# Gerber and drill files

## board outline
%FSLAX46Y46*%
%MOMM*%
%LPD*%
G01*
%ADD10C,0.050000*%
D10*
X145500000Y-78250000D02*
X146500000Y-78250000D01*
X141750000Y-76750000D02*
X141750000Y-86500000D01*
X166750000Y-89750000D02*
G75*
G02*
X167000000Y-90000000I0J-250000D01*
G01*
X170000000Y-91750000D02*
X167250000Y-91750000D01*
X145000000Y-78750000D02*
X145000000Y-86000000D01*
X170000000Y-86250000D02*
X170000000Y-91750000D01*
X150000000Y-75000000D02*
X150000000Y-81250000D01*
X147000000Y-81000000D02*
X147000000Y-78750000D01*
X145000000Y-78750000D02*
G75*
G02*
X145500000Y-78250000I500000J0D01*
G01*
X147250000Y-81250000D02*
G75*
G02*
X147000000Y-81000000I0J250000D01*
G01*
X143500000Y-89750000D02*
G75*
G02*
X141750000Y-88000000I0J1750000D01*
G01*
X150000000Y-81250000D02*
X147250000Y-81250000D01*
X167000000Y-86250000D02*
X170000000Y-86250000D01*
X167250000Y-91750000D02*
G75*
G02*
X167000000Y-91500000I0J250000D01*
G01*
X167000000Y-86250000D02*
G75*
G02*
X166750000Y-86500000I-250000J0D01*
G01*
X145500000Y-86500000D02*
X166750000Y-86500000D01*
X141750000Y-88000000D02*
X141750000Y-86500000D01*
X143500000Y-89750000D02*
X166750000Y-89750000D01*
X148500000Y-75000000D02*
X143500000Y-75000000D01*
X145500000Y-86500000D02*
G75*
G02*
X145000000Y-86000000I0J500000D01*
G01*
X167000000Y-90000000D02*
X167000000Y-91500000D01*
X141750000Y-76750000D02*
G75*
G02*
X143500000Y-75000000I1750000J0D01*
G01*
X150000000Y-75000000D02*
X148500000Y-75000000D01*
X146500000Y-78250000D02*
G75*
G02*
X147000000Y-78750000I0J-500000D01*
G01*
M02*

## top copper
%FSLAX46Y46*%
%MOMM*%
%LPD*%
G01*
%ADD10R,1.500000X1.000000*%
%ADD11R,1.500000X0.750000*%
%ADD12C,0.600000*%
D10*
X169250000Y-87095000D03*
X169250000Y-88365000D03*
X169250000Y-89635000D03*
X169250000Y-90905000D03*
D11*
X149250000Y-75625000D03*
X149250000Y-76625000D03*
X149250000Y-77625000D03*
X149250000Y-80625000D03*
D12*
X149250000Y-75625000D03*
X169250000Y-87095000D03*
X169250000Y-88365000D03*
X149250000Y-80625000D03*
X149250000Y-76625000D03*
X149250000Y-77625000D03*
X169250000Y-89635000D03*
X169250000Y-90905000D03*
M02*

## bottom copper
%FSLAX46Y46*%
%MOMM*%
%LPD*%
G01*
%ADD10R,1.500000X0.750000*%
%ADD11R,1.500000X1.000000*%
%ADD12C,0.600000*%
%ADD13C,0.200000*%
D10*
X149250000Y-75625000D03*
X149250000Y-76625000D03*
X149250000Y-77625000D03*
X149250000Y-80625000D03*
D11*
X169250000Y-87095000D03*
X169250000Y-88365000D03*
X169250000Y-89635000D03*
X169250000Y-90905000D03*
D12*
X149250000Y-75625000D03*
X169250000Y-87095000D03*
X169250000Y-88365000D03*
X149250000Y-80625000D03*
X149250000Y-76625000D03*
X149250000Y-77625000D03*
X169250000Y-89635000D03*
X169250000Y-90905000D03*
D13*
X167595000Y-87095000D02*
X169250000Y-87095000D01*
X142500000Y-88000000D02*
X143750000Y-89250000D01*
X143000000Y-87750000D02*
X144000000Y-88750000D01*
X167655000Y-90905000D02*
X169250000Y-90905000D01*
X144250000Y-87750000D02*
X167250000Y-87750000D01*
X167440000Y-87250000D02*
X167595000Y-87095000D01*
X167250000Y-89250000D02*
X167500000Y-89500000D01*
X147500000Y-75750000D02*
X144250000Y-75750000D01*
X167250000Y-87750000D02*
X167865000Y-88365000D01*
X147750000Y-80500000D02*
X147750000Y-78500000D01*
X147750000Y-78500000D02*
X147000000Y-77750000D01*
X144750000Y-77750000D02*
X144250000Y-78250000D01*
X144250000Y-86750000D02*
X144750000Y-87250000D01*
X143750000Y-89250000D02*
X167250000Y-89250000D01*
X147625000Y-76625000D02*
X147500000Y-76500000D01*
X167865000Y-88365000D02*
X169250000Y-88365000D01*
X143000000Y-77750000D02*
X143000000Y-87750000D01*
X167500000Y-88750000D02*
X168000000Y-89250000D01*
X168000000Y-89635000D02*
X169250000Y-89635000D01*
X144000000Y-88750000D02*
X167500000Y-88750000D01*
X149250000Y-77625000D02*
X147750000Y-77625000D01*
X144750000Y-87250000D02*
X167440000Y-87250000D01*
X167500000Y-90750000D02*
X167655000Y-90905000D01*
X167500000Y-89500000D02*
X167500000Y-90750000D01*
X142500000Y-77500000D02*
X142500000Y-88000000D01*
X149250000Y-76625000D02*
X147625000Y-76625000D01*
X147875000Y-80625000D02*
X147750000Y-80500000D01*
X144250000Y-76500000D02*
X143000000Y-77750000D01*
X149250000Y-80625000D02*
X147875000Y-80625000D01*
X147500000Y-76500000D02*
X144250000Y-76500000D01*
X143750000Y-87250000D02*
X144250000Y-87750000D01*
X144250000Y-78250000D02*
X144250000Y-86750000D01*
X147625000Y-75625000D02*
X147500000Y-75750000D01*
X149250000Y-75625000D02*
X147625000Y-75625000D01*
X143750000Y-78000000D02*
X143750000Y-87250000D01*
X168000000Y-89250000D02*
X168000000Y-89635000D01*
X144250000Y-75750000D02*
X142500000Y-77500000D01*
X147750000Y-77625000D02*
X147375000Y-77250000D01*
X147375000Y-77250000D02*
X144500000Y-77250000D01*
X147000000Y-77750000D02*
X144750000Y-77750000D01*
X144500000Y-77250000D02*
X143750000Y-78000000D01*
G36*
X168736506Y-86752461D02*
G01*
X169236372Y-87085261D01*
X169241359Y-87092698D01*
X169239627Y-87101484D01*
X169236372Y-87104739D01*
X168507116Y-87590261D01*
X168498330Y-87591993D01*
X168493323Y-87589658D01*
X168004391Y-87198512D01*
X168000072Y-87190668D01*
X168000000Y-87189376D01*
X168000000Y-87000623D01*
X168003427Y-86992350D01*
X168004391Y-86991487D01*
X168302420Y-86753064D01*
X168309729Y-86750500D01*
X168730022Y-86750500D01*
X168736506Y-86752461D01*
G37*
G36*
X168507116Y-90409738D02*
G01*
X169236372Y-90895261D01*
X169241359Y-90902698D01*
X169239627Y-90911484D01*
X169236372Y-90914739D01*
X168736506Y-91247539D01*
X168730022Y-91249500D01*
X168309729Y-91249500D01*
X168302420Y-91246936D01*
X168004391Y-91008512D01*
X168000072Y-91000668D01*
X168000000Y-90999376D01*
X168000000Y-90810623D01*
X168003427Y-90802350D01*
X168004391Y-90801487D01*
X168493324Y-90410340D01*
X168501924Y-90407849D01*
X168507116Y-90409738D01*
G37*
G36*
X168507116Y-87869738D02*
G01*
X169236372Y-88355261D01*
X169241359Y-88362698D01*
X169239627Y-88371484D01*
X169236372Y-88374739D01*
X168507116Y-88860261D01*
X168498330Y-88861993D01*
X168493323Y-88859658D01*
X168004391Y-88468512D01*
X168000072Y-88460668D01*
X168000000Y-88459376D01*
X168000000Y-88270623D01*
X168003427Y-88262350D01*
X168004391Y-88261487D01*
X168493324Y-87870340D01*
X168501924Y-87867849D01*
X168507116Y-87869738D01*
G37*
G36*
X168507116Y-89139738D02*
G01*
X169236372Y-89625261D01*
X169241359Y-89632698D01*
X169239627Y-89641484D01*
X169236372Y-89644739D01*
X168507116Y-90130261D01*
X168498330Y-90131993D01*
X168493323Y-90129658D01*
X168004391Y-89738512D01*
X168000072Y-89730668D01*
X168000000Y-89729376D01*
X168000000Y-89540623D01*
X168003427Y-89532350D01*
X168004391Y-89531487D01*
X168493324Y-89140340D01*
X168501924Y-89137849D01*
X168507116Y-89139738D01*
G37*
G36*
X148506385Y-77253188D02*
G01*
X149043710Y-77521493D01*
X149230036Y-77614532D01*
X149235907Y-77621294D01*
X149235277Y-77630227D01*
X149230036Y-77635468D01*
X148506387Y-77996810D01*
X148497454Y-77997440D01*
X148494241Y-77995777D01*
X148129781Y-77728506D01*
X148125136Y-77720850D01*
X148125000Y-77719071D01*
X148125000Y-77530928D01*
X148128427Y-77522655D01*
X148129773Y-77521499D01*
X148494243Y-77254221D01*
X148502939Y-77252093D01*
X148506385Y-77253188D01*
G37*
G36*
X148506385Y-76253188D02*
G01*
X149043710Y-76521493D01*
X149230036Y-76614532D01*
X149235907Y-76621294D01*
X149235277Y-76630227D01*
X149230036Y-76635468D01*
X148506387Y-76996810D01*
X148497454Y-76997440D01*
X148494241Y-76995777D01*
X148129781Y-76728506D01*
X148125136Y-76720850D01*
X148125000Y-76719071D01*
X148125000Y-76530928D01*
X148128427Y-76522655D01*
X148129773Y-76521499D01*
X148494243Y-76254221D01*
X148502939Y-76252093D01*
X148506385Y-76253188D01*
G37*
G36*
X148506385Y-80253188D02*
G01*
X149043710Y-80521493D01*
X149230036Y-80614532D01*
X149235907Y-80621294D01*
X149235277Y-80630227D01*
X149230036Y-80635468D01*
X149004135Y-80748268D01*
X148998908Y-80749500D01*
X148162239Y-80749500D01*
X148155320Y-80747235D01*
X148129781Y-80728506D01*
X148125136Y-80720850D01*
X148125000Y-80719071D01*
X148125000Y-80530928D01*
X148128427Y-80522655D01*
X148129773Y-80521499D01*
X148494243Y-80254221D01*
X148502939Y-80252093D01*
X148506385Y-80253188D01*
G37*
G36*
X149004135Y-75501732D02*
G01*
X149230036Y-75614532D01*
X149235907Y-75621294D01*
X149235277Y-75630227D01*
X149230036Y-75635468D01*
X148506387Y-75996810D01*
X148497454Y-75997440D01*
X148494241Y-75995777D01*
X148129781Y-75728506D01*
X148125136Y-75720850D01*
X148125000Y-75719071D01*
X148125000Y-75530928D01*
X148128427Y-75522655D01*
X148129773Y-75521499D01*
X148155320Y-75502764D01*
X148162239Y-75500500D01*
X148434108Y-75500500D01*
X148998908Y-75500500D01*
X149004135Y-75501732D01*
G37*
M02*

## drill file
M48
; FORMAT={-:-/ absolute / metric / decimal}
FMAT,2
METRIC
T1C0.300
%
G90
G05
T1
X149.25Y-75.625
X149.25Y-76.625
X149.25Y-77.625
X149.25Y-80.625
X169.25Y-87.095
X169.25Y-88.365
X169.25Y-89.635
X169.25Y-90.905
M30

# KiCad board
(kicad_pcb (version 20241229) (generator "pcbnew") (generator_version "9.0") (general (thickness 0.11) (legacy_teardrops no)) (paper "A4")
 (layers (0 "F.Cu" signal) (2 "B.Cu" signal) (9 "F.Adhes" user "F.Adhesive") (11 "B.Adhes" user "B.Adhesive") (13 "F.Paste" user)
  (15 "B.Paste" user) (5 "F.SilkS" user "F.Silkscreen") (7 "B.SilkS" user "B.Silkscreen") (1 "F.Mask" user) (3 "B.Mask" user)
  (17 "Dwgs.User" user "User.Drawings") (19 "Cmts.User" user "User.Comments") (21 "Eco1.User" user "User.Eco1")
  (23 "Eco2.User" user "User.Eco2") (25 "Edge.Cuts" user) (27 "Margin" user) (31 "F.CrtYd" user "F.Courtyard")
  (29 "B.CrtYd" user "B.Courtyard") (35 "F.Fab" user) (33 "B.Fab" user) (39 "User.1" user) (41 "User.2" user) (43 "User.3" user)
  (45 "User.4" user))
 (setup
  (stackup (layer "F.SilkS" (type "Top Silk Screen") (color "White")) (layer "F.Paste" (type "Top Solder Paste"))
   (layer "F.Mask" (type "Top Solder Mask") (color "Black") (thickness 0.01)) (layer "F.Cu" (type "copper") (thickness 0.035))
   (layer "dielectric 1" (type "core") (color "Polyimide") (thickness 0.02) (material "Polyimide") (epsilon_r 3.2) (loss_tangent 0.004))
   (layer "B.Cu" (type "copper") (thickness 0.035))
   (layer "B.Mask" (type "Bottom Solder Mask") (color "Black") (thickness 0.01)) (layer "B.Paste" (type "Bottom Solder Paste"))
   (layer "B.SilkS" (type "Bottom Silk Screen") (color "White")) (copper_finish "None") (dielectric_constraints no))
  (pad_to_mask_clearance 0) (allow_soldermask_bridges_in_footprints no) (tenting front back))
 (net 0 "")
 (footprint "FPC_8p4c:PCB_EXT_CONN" (layer "F.Cu") (at 169.25 89)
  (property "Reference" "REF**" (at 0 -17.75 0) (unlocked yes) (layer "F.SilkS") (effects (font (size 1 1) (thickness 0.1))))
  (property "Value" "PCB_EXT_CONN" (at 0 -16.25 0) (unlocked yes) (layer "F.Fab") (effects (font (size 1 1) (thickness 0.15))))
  (pad "1" smd rect (at 0 -1.905) (size 1.5 1) (layers "F.Cu" "F.Mask" "F.Paste")
   (teardrops (best_length_ratio 0.5) (max_length 1) (best_width_ratio 1) (max_width 2) (curved_edges no) (filter_ratio 0.9) (enabled yes)
    (allow_two_segments yes) (prefer_zone_connections yes)))
  (pad "2" smd rect (at 0 -0.635) (size 1.5 1) (layers "F.Cu" "F.Mask" "F.Paste")
   (teardrops (best_length_ratio 0.5) (max_length 1) (best_width_ratio 1) (max_width 2) (curved_edges no) (filter_ratio 0.9) (enabled yes)
    (allow_two_segments yes) (prefer_zone_connections yes)))
  (pad "3" smd rect (at 0 0.635) (size 1.5 1) (layers "F.Cu" "F.Mask" "F.Paste")
   (teardrops (best_length_ratio 0.5) (max_length 1) (best_width_ratio 1) (max_width 2) (curved_edges no) (filter_ratio 0.9) (enabled yes)
    (allow_two_segments yes) (prefer_zone_connections yes)))
  (pad "4" smd rect (at 0 1.905) (size 1.5 1) (layers "F.Cu" "F.Mask" "F.Paste")
   (teardrops (best_length_ratio 0.5) (max_length 1) (best_width_ratio 1) (max_width 2) (curved_edges no) (filter_ratio 0.9) (enabled yes)
    (allow_two_segments yes) (prefer_zone_connections yes))))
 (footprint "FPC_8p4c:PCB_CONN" (layer "F.Cu") (at 149.25 78.125)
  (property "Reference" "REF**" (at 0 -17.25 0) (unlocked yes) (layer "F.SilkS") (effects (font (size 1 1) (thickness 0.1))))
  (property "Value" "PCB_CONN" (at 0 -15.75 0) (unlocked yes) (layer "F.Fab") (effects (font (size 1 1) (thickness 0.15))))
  (pad "1" smd rect (at 0 -2.5) (size 1.5 0.75) (layers "F.Cu" "F.Mask" "F.Paste")
   (teardrops (best_length_ratio 0.5) (max_length 1) (best_width_ratio 1) (max_width 2) (curved_edges no) (filter_ratio 0.9) (enabled yes)
    (allow_two_segments yes) (prefer_zone_connections yes)))
  (pad "2" smd rect (at 0 -1.5) (size 1.5 0.75) (layers "F.Cu" "F.Mask" "F.Paste")
   (teardrops (best_length_ratio 0.5) (max_length 1) (best_width_ratio 1) (max_width 2) (curved_edges no) (filter_ratio 0.9) (enabled yes)
    (allow_two_segments yes) (prefer_zone_connections yes)))
  (pad "3" smd rect (at 0 -0.5) (size 1.5 0.75) (layers "F.Cu" "F.Mask" "F.Paste")
   (teardrops (best_length_ratio 0.5) (max_length 1) (best_width_ratio 1) (max_width 2) (curved_edges no) (filter_ratio 0.9) (enabled yes)
    (allow_two_segments yes) (prefer_zone_connections yes)))
  (pad "4" smd rect (at 0 2.5) (size 1.5 0.75) (layers "F.Cu" "F.Mask" "F.Paste")
   (teardrops (best_length_ratio 0.5) (max_length 1) (best_width_ratio 1) (max_width 2) (curved_edges no) (filter_ratio 0.9) (enabled yes)
    (allow_two_segments yes) (prefer_zone_connections yes))))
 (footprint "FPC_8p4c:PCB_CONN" (layer "B.Cu") (at 149.25 78.125 180)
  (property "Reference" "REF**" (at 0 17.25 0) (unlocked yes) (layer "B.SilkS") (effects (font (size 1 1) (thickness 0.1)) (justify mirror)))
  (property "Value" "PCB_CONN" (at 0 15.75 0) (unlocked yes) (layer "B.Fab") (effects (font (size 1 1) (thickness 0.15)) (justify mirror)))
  (pad "1" smd rect (at 0 2.5 180) (size 1.5 0.75) (layers "B.Cu" "B.Mask" "B.Paste")
   (teardrops (best_length_ratio 0.5) (max_length 1) (best_width_ratio 1) (max_width 2) (curved_edges no) (filter_ratio 0.9) (enabled yes)
    (allow_two_segments yes) (prefer_zone_connections yes)))
  (pad "2" smd rect (at 0 1.5 180) (size 1.5 0.75) (layers "B.Cu" "B.Mask" "B.Paste")
   (teardrops (best_length_ratio 0.5) (max_length 1) (best_width_ratio 1) (max_width 2) (curved_edges no) (filter_ratio 0.9) (enabled yes)
    (allow_two_segments yes) (prefer_zone_connections yes)))
  (pad "3" smd rect (at 0 0.5 180) (size 1.5 0.75) (layers "B.Cu" "B.Mask" "B.Paste")
   (teardrops (best_length_ratio 0.5) (max_length 1) (best_width_ratio 1) (max_width 2) (curved_edges no) (filter_ratio 0.9) (enabled yes)
    (allow_two_segments yes) (prefer_zone_connections yes)))
  (pad "4" smd rect (at 0 -2.5 180) (size 1.5 0.75) (layers "B.Cu" "B.Mask" "B.Paste")
   (teardrops (best_length_ratio 0.5) (max_length 1) (best_width_ratio 1) (max_width 2) (curved_edges no) (filter_ratio 0.9) (enabled yes)
    (allow_two_segments yes) (prefer_zone_connections yes))))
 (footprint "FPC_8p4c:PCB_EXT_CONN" (layer "B.Cu") (at 169.25 89 180)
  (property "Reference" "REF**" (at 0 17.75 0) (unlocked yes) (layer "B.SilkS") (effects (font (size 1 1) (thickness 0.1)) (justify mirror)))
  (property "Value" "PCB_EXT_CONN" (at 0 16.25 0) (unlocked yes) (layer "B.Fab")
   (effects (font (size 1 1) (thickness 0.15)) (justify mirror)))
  (pad "1" smd rect (at 0 1.905 180) (size 1.5 1) (layers "B.Cu" "B.Mask" "B.Paste")
   (teardrops (best_length_ratio 0.5) (max_length 1) (best_width_ratio 1) (max_width 2) (curved_edges no) (filter_ratio 0.9) (enabled yes)
    (allow_two_segments yes) (prefer_zone_connections yes)))
  (pad "2" smd rect (at 0 0.635 180) (size 1.5 1) (layers "B.Cu" "B.Mask" "B.Paste")
   (teardrops (best_length_ratio 0.5) (max_length 1) (best_width_ratio 1) (max_width 2) (curved_edges no) (filter_ratio 0.9) (enabled yes)
    (allow_two_segments yes) (prefer_zone_connections yes)))
  (pad "3" smd rect (at 0 -0.635 180) (size 1.5 1) (layers "B.Cu" "B.Mask" "B.Paste")
   (teardrops (best_length_ratio 0.5) (max_length 1) (best_width_ratio 1) (max_width 2) (curved_edges no) (filter_ratio 0.9) (enabled yes)
    (allow_two_segments yes) (prefer_zone_connections yes)))
  (pad "4" smd rect (at 0 -1.905 180) (size 1.5 1) (layers "B.Cu" "B.Mask" "B.Paste")
   (teardrops (best_length_ratio 0.5) (max_length 1) (best_width_ratio 1) (max_width 2) (curved_edges no) (filter_ratio 0.9) (enabled yes)
    (allow_two_segments yes) (prefer_zone_connections yes))))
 (gr_line (start 145.5 78.25) (end 146.5 78.25) (stroke (width 0.05) (type default)) (layer "Edge.Cuts"))
 (gr_line (start 141.75 76.75) (end 141.75 86.5) (stroke (width 0.05) (type default)) (layer "Edge.Cuts"))
 (gr_arc (start 166.75 89.75) (mid 166.926777 89.823223) (end 167 90) (stroke (width 0.05) (type default)) (layer "Edge.Cuts"))
 (gr_line (start 170 91.75) (end 167.25 91.75) (stroke (width 0.05) (type default)) (layer "Edge.Cuts"))
 (gr_line (start 145 78.75) (end 145 86) (stroke (width 0.05) (type default)) (layer "Edge.Cuts"))
 (gr_line (start 170 86.25) (end 170 91.75) (stroke (width 0.05) (type default)) (layer "Edge.Cuts"))
 (gr_line (start 150 75) (end 150 81.25) (stroke (width 0.05) (type default)) (layer "Edge.Cuts"))
 (gr_line (start 147 81) (end 147 78.75) (stroke (width 0.05) (type default)) (layer "Edge.Cuts"))
 (gr_arc (start 145 78.75) (mid 145.146447 78.396447) (end 145.5 78.25) (stroke (width 0.05) (type default)) (layer "Edge.Cuts"))
 (gr_arc (start 147.25 81.25) (mid 147.073223 81.176777) (end 147 81) (stroke (width 0.05) (type default)) (layer "Edge.Cuts"))
 (gr_arc (start 143.5 89.75) (mid 142.262563 89.237437) (end 141.75 88) (stroke (width 0.05) (type default)) (layer "Edge.Cuts"))
 (gr_line (start 150 81.25) (end 147.25 81.25) (stroke (width 0.05) (type default)) (layer "Edge.Cuts"))
 (gr_line (start 167 86.25) (end 170 86.25) (stroke (width 0.05) (type default)) (layer "Edge.Cuts"))
 (gr_arc (start 167.25 91.75) (mid 167.073223 91.676777) (end 167 91.5) (stroke (width 0.05) (type default)) (layer "Edge.Cuts"))
 (gr_arc (start 167 86.25) (mid 166.926777 86.426777) (end 166.75 86.5) (stroke (width 0.05) (type default)) (layer "Edge.Cuts"))
 (gr_line (start 145.5 86.5) (end 166.75 86.5) (stroke (width 0.05) (type default)) (layer "Edge.Cuts"))
 (gr_line (start 141.75 88) (end 141.75 86.5) (stroke (width 0.05) (type default)) (layer "Edge.Cuts"))
 (gr_line (start 143.5 89.75) (end 166.75 89.75) (stroke (width 0.05) (type default)) (layer "Edge.Cuts"))
 (gr_line (start 148.5 75) (end 143.5 75) (stroke (width 0.05) (type default)) (layer "Edge.Cuts"))
 (gr_arc (start 145.5 86.5) (mid 145.146447 86.353553) (end 145 86) (stroke (width 0.05) (type default)) (layer "Edge.Cuts"))
 (gr_line (start 167 90) (end 167 91.5) (stroke (width 0.05) (type default)) (layer "Edge.Cuts"))
 (gr_arc (start 141.75 76.75) (mid 142.262563 75.512563) (end 143.5 75) (stroke (width 0.05) (type default)) (layer "Edge.Cuts"))
 (gr_line (start 150 75) (end 148.5 75) (stroke (width 0.05) (type default)) (layer "Edge.Cuts"))
 (gr_arc (start 146.5 78.25) (mid 146.853553 78.396447) (end 147 78.75) (stroke (width 0.05) (type default)) (layer "Edge.Cuts"))
 (via (at 149.25 75.625) (size 0.6) (drill 0.3) (layers "F.Cu" "B.Cu") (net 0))
 (via (at 169.25 87.095) (size 0.6) (drill 0.3) (layers "F.Cu" "B.Cu") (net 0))
 (via (at 169.25 88.365) (size 0.6) (drill 0.3) (layers "F.Cu" "B.Cu") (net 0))
 (via (at 149.25 80.625) (size 0.6) (drill 0.3) (layers "F.Cu" "B.Cu") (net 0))
 (via (at 149.25 76.625) (size 0.6) (drill 0.3) (layers "F.Cu" "B.Cu") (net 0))
 (via (at 149.25 77.625) (size 0.6) (drill 0.3) (layers "F.Cu" "B.Cu") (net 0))
 (via (at 169.25 89.635) (size 0.6) (drill 0.3) (layers "F.Cu" "B.Cu") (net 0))
 (via (at 169.25 90.905) (size 0.6) (drill 0.3) (layers "F.Cu" "B.Cu") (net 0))
 (segment (start 167.595 87.095) (end 169.25 87.095) (width 0.2) (layer "B.Cu") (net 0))
 (segment (start 142.5 88) (end 143.75 89.25) (width 0.2) (layer "B.Cu") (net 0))
 (segment (start 143 87.75) (end 144 88.75) (width 0.2) (layer "B.Cu") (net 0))
 (segment (start 167.655 90.905) (end 169.25 90.905) (width 0.2) (layer "B.Cu") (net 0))
 (segment (start 144.25 87.75) (end 167.25 87.75) (width 0.2) (layer "B.Cu") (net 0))
 (segment (start 167.44 87.25) (end 167.595 87.095) (width 0.2) (layer "B.Cu") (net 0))
 (segment (start 167.25 89.25) (end 167.5 89.5) (width 0.2) (layer "B.Cu") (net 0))
 (segment (start 147.5 75.75) (end 144.25 75.75) (width 0.2) (layer "B.Cu") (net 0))
 (segment (start 167.25 87.75) (end 167.865 88.365) (width 0.2) (layer "B.Cu") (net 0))
 (segment (start 147.75 80.5) (end 147.75 78.5) (width 0.2) (layer "B.Cu") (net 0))
 (segment (start 147.75 78.5) (end 147 77.75) (width 0.2) (layer "B.Cu") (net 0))
 (segment (start 144.75 77.75) (end 144.25 78.25) (width 0.2) (layer "B.Cu") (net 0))
 (segment (start 144.25 86.75) (end 144.75 87.25) (width 0.2) (layer "B.Cu") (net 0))
 (segment (start 143.75 89.25) (end 167.25 89.25) (width 0.2) (layer "B.Cu") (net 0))
 (segment (start 147.625 76.625) (end 147.5 76.5) (width 0.2) (layer "B.Cu") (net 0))
 (segment (start 167.865 88.365) (end 169.25 88.365) (width 0.2) (layer "B.Cu") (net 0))
 (segment (start 143 77.75) (end 143 87.75) (width 0.2) (layer "B.Cu") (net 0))
 (segment (start 167.5 88.75) (end 168 89.25) (width 0.2) (layer "B.Cu") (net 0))
 (segment (start 168 89.635) (end 169.25 89.635) (width 0.2) (layer "B.Cu") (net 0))
 (segment (start 144 88.75) (end 167.5 88.75) (width 0.2) (layer "B.Cu") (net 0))
 (segment (start 149.25 77.625) (end 147.75 77.625) (width 0.2) (layer "B.Cu") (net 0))
 (segment (start 144.75 87.25) (end 167.44 87.25) (width 0.2) (layer "B.Cu") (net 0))
 (segment (start 167.5 90.75) (end 167.655 90.905) (width 0.2) (layer "B.Cu") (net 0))
 (segment (start 167.5 89.5) (end 167.5 90.75) (width 0.2) (layer "B.Cu") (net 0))
 (segment (start 142.5 77.5) (end 142.5 88) (width 0.2) (layer "B.Cu") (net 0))
 (segment (start 149.25 76.625) (end 147.625 76.625) (width 0.2) (layer "B.Cu") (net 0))
 (segment (start 147.875 80.625) (end 147.75 80.5) (width 0.2) (layer "B.Cu") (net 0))
 (segment (start 144.25 76.5) (end 143 77.75) (width 0.2) (layer "B.Cu") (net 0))
 (segment (start 149.25 80.625) (end 147.875 80.625) (width 0.2) (layer "B.Cu") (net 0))
 (segment (start 147.5 76.5) (end 144.25 76.5) (width 0.2) (layer "B.Cu") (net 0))
 (segment (start 143.75 87.25) (end 144.25 87.75) (width 0.2) (layer "B.Cu") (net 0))
 (segment (start 144.25 78.25) (end 144.25 86.75) (width 0.2) (layer "B.Cu") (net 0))
 (segment (start 147.625 75.625) (end 147.5 75.75) (width 0.2) (layer "B.Cu") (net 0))
 (segment (start 149.25 75.625) (end 147.625 75.625) (width 0.2) (layer "B.Cu") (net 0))
 (segment (start 143.75 78) (end 143.75 87.25) (width 0.2) (layer "B.Cu") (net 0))
 (segment (start 168 89.25) (end 168 89.635) (width 0.2) (layer "B.Cu") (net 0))
 (segment (start 144.25 75.75) (end 142.5 77.5) (width 0.2) (layer "B.Cu") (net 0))
 (segment (start 147.75 77.625) (end 147.375 77.25) (width 0.2) (layer "B.Cu") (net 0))
 (segment (start 147.375 77.25) (end 144.5 77.25) (width 0.2) (layer "B.Cu") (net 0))
 (segment (start 147 77.75) (end 144.75 77.75) (width 0.2) (layer "B.Cu") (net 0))
 (segment (start 144.5 77.25) (end 143.75 78) (width 0.2) (layer "B.Cu") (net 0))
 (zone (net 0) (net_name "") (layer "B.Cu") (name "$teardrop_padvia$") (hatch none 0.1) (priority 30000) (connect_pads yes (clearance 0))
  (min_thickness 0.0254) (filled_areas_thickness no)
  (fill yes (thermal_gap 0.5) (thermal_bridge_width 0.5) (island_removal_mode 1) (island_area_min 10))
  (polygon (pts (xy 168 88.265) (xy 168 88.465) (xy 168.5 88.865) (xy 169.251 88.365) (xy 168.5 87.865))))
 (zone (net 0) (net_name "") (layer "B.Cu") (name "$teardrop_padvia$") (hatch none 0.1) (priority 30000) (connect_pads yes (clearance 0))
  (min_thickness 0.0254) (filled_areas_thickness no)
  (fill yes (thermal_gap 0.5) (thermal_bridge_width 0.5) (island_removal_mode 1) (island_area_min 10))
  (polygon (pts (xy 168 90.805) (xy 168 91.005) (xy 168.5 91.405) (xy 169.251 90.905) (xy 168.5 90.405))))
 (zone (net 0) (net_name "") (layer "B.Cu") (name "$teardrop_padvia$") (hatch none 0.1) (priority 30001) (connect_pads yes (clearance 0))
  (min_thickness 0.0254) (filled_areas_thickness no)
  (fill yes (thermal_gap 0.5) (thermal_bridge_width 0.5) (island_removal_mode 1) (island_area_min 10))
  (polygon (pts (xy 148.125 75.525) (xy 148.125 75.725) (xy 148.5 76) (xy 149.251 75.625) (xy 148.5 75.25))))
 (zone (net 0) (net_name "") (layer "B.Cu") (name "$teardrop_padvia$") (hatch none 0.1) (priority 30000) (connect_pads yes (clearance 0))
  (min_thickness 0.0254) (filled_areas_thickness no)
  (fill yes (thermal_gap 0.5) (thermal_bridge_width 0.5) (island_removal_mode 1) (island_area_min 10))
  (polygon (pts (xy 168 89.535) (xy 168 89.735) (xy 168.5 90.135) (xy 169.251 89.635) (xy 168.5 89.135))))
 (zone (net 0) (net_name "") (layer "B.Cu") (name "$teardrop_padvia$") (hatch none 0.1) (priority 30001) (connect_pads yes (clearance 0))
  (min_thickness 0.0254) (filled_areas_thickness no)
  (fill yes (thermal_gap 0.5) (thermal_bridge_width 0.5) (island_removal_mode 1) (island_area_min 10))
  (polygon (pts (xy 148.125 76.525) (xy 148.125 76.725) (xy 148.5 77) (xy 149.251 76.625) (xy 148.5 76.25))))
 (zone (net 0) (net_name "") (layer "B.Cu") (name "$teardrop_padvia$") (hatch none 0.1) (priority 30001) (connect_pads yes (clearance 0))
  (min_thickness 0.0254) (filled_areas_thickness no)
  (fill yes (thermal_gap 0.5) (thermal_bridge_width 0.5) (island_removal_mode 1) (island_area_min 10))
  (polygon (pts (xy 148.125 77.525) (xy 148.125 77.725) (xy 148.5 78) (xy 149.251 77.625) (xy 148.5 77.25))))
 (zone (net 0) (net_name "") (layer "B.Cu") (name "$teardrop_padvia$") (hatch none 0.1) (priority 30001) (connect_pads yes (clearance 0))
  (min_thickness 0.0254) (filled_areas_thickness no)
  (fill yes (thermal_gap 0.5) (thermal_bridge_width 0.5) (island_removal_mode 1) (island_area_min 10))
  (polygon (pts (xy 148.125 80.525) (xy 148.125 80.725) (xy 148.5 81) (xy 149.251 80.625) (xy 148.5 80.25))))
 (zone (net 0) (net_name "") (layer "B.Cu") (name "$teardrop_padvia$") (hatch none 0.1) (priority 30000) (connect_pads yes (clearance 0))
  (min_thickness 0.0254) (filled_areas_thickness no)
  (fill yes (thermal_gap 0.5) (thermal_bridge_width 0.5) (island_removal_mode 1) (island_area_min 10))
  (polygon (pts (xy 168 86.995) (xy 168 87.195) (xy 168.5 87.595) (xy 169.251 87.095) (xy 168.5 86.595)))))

